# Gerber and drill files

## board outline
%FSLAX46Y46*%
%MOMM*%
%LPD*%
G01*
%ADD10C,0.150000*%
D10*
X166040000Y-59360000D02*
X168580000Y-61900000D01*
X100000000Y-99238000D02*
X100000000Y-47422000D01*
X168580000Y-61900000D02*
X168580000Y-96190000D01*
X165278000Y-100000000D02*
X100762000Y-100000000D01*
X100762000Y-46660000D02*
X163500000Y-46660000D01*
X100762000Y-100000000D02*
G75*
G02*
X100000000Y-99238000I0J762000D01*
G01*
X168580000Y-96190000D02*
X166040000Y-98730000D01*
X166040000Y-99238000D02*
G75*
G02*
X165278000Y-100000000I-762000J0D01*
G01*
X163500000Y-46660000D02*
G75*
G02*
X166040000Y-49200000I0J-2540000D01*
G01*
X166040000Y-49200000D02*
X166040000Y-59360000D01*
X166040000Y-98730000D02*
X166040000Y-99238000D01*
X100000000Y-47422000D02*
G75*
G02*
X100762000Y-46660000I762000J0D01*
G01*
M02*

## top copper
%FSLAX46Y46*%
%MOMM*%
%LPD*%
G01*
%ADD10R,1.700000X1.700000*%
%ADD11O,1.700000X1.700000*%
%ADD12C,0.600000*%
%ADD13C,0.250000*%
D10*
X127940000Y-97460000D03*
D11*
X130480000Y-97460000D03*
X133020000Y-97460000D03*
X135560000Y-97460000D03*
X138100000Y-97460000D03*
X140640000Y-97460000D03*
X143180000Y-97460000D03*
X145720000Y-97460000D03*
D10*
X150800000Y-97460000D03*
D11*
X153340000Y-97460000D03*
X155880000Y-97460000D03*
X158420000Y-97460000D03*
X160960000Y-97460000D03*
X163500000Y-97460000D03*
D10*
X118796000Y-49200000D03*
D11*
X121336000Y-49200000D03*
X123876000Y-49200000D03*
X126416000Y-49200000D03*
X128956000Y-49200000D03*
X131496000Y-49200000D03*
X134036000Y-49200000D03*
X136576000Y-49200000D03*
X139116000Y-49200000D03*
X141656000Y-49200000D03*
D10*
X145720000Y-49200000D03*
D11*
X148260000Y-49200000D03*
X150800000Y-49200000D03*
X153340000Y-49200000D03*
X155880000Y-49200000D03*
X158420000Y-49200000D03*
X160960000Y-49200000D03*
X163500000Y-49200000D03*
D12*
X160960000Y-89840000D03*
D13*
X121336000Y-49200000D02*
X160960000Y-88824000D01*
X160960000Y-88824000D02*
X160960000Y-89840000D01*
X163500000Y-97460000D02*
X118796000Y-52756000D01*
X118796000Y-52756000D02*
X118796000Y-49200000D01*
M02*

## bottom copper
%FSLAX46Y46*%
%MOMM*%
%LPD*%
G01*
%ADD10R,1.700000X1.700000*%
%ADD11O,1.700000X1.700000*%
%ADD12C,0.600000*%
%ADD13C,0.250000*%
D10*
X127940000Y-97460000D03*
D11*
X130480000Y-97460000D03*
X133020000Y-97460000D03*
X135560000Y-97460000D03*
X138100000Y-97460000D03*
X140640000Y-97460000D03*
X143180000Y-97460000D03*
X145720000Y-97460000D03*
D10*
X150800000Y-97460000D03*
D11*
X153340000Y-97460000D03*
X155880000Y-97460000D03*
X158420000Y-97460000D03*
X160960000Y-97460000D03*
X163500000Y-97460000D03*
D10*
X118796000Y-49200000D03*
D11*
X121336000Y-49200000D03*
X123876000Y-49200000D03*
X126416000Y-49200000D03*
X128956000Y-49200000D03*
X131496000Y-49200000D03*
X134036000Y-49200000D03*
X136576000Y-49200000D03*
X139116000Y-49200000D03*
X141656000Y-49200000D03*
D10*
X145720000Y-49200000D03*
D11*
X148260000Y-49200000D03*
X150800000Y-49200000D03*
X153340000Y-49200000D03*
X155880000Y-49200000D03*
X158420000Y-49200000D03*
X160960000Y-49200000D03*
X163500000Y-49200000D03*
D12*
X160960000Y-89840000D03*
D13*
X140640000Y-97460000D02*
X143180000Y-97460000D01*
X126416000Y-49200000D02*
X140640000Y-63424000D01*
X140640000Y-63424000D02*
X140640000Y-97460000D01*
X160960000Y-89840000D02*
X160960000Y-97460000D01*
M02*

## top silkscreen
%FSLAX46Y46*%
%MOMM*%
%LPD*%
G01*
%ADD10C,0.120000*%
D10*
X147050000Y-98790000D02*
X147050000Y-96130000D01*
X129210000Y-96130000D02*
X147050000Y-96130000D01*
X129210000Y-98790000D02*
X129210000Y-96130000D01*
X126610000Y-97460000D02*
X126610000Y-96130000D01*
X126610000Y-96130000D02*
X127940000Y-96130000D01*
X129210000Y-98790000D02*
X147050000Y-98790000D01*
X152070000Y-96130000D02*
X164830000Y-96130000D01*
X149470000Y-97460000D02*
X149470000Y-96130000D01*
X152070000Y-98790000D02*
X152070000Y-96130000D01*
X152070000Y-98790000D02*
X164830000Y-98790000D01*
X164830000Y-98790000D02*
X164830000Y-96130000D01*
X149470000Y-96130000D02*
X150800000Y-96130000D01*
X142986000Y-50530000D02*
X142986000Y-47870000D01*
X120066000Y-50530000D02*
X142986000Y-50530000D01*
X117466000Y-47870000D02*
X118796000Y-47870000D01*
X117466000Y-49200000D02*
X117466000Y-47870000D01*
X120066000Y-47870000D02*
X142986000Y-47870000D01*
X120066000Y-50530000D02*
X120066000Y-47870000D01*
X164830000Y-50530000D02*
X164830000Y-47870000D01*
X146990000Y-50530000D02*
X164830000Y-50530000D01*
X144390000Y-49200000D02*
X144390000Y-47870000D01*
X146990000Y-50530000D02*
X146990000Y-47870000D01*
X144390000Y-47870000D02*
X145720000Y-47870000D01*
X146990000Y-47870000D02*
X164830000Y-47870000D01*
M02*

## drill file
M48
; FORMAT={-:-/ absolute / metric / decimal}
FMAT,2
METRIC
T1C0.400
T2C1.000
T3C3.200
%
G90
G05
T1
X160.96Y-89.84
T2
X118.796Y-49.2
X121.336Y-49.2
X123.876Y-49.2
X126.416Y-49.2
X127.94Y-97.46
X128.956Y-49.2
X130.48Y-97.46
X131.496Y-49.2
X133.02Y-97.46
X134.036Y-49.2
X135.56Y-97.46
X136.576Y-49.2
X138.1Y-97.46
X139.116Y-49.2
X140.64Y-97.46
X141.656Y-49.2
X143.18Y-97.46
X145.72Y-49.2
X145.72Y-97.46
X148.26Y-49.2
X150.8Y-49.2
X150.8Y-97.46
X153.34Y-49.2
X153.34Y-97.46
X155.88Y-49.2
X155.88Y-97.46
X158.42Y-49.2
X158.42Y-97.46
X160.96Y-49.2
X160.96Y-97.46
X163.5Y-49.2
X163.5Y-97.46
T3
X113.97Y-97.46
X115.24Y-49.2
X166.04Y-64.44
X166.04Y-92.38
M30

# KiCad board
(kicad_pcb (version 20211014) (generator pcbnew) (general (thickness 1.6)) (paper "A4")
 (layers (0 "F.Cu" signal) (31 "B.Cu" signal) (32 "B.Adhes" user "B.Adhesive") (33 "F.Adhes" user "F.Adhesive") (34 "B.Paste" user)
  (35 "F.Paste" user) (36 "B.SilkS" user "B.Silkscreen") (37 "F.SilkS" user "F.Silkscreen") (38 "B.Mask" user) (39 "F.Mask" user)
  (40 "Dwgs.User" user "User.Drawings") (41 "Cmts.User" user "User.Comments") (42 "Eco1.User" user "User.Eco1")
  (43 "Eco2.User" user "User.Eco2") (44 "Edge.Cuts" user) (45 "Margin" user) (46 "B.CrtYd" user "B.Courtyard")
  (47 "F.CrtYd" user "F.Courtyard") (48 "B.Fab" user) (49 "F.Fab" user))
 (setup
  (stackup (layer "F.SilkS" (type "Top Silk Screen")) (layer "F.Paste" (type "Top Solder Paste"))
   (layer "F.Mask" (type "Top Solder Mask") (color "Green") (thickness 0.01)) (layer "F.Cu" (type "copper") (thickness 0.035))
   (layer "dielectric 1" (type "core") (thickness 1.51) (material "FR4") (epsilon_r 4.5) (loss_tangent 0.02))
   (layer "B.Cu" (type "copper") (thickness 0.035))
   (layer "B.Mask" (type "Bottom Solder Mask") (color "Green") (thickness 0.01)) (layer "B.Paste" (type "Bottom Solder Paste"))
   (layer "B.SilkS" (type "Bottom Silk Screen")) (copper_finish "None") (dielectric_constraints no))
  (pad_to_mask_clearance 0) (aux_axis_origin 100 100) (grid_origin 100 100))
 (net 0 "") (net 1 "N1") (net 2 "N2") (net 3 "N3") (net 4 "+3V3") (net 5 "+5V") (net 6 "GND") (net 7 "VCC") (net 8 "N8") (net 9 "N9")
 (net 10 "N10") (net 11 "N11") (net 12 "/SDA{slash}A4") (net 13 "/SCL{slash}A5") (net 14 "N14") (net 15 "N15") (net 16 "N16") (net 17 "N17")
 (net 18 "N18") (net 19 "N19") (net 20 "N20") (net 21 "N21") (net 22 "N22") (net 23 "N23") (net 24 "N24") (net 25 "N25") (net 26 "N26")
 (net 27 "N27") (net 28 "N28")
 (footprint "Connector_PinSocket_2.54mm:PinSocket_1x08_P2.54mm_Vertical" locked (layer "F.Cu") (at 127.94 97.46 90)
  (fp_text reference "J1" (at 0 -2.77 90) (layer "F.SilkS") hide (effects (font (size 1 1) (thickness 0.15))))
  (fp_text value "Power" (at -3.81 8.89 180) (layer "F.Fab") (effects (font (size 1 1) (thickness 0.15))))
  (fp_line (start -1.33 19.11) (end 1.33 19.11) (layer "F.SilkS") (width 0.12))
  (fp_line (start 1.33 1.27) (end 1.33 19.11) (layer "F.SilkS") (width 0.12))
  (fp_line (start -1.33 1.27) (end 1.33 1.27) (layer "F.SilkS") (width 0.12))
  (fp_line (start 0 -1.33) (end 1.33 -1.33) (layer "F.SilkS") (width 0.12))
  (fp_line (start 1.33 -1.33) (end 1.33 0) (layer "F.SilkS") (width 0.12))
  (fp_line (start -1.33 1.27) (end -1.33 19.11) (layer "F.SilkS") (width 0.12))
  (pad "1" thru_hole rect locked (at 0 0 90) (size 1.7 1.7) (drill 1) (layers *.Cu *.Mask) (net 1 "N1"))
  (pad "2" thru_hole oval locked (at 0 2.54 90) (size 1.7 1.7) (drill 1) (layers *.Cu *.Mask) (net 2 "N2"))
  (pad "3" thru_hole oval locked (at 0 5.08 90) (size 1.7 1.7) (drill 1) (layers *.Cu *.Mask) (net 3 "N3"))
  (pad "4" thru_hole oval locked (at 0 7.62 90) (size 1.7 1.7) (drill 1) (layers *.Cu *.Mask) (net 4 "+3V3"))
  (pad "5" thru_hole oval locked (at 0 10.16 90) (size 1.7 1.7) (drill 1) (layers *.Cu *.Mask) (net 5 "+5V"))
  (pad "6" thru_hole oval locked (at 0 12.7 90) (size 1.7 1.7) (drill 1) (layers *.Cu *.Mask) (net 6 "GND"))
  (pad "7" thru_hole oval locked (at 0 15.24 90) (size 1.7 1.7) (drill 1) (layers *.Cu *.Mask) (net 6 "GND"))
  (pad "8" thru_hole oval locked (at 0 17.78 90) (size 1.7 1.7) (drill 1) (layers *.Cu *.Mask) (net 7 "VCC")))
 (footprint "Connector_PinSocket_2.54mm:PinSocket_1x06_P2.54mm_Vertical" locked (layer "F.Cu") (at 150.8 97.46 90)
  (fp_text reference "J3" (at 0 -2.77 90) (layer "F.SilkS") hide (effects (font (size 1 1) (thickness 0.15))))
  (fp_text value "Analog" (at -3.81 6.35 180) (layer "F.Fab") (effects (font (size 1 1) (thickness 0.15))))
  (fp_line (start 1.33 1.27) (end 1.33 14.03) (layer "F.SilkS") (width 0.12))
  (fp_line (start 0 -1.33) (end 1.33 -1.33) (layer "F.SilkS") (width 0.12))
  (fp_line (start -1.33 1.27) (end 1.33 1.27) (layer "F.SilkS") (width 0.12))
  (fp_line (start -1.33 1.27) (end -1.33 14.03) (layer "F.SilkS") (width 0.12))
  (fp_line (start -1.33 14.03) (end 1.33 14.03) (layer "F.SilkS") (width 0.12))
  (fp_line (start 1.33 -1.33) (end 1.33 0) (layer "F.SilkS") (width 0.12))
  (pad "1" thru_hole rect locked (at 0 0 90) (size 1.7 1.7) (drill 1) (layers *.Cu *.Mask) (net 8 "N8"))
  (pad "2" thru_hole oval locked (at 0 2.54 90) (size 1.7 1.7) (drill 1) (layers *.Cu *.Mask) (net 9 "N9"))
  (pad "3" thru_hole oval locked (at 0 5.08 90) (size 1.7 1.7) (drill 1) (layers *.Cu *.Mask) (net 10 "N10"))
  (pad "4" thru_hole oval locked (at 0 7.62 90) (size 1.7 1.7) (drill 1) (layers *.Cu *.Mask) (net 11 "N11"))
  (pad "5" thru_hole oval locked (at 0 10.16 90) (size 1.7 1.7) (drill 1) (layers *.Cu *.Mask) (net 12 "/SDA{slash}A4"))
  (pad "6" thru_hole oval locked (at 0 12.7 90) (size 1.7 1.7) (drill 1) (layers *.Cu *.Mask) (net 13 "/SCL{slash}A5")))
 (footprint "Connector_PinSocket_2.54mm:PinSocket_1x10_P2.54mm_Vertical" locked (layer "F.Cu") (at 118.796 49.2 90)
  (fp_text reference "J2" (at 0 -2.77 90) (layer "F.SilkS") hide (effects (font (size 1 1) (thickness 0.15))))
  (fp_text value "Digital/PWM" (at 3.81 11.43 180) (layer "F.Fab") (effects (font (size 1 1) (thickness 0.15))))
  (fp_line (start -1.33 24.19) (end 1.33 24.19) (layer "F.SilkS") (width 0.12))
  (fp_line (start -1.33 1.27) (end -1.33 24.19) (layer "F.SilkS") (width 0.12))
  (fp_line (start 1.33 -1.33) (end 1.33 0) (layer "F.SilkS") (width 0.12))
  (fp_line (start 0 -1.33) (end 1.33 -1.33) (layer "F.SilkS") (width 0.12))
  (fp_line (start 1.33 1.27) (end 1.33 24.19) (layer "F.SilkS") (width 0.12))
  (fp_line (start -1.33 1.27) (end 1.33 1.27) (layer "F.SilkS") (width 0.12))
  (pad "1" thru_hole rect locked (at 0 0 90) (size 1.7 1.7) (drill 1) (layers *.Cu *.Mask) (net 13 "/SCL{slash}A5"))
  (pad "2" thru_hole oval locked (at 0 2.54 90) (size 1.7 1.7) (drill 1) (layers *.Cu *.Mask) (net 12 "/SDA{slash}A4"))
  (pad "3" thru_hole oval locked (at 0 5.08 90) (size 1.7 1.7) (drill 1) (layers *.Cu *.Mask) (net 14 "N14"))
  (pad "4" thru_hole oval locked (at 0 7.62 90) (size 1.7 1.7) (drill 1) (layers *.Cu *.Mask) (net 6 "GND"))
  (pad "5" thru_hole oval locked (at 0 10.16 90) (size 1.7 1.7) (drill 1) (layers *.Cu *.Mask) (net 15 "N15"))
  (pad "6" thru_hole oval locked (at 0 12.7 90) (size 1.7 1.7) (drill 1) (layers *.Cu *.Mask) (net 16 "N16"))
  (pad "7" thru_hole oval locked (at 0 15.24 90) (size 1.7 1.7) (drill 1) (layers *.Cu *.Mask) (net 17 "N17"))
  (pad "8" thru_hole oval locked (at 0 17.78 90) (size 1.7 1.7) (drill 1) (layers *.Cu *.Mask) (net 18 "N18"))
  (pad "9" thru_hole oval locked (at 0 20.32 90) (size 1.7 1.7) (drill 1) (layers *.Cu *.Mask) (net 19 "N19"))
  (pad "10" thru_hole oval locked (at 0 22.86 90) (size 1.7 1.7) (drill 1) (layers *.Cu *.Mask) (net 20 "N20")))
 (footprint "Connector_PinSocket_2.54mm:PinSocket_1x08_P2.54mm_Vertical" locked (layer "F.Cu") (at 145.72 49.2 90)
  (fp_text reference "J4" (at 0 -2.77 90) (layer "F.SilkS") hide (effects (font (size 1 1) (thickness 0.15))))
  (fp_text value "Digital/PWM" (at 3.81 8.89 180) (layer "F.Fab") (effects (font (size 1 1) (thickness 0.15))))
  (fp_line (start -1.33 19.11) (end 1.33 19.11) (layer "F.SilkS") (width 0.12))
  (fp_line (start -1.33 1.27) (end -1.33 19.11) (layer "F.SilkS") (width 0.12))
  (fp_line (start 0 -1.33) (end 1.33 -1.33) (layer "F.SilkS") (width 0.12))
  (fp_line (start -1.33 1.27) (end 1.33 1.27) (layer "F.SilkS") (width 0.12))
  (fp_line (start 1.33 -1.33) (end 1.33 0) (layer "F.SilkS") (width 0.12))
  (fp_line (start 1.33 1.27) (end 1.33 19.11) (layer "F.SilkS") (width 0.12))
  (pad "1" thru_hole rect locked (at 0 0 90) (size 1.7 1.7) (drill 1) (layers *.Cu *.Mask) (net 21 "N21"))
  (pad "2" thru_hole oval locked (at 0 2.54 90) (size 1.7 1.7) (drill 1) (layers *.Cu *.Mask) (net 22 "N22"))
  (pad "3" thru_hole oval locked (at 0 5.08 90) (size 1.7 1.7) (drill 1) (layers *.Cu *.Mask) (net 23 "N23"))
  (pad "4" thru_hole oval locked (at 0 7.62 90) (size 1.7 1.7) (drill 1) (layers *.Cu *.Mask) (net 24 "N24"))
  (pad "5" thru_hole oval locked (at 0 10.16 90) (size 1.7 1.7) (drill 1) (layers *.Cu *.Mask) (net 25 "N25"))
  (pad "6" thru_hole oval locked (at 0 12.7 90) (size 1.7 1.7) (drill 1) (layers *.Cu *.Mask) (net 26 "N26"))
  (pad "7" thru_hole oval locked (at 0 15.24 90) (size 1.7 1.7) (drill 1) (layers *.Cu *.Mask) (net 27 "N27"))
  (pad "8" thru_hole oval locked (at 0 17.78 90) (size 1.7 1.7) (drill 1) (layers *.Cu *.Mask) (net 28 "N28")))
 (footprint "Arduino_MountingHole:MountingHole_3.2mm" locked (layer "F.Cu") (at 115.24 49.2)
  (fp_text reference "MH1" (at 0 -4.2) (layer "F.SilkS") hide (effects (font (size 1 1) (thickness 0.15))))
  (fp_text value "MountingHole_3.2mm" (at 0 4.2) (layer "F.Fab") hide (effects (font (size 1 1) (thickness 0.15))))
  (pad "" np_thru_hole circle locked (at 0 0) (size 3.2 3.2) (drill 3.2) (layers *.Cu *.Mask)))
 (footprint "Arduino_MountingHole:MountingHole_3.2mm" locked (layer "F.Cu") (at 113.97 97.46)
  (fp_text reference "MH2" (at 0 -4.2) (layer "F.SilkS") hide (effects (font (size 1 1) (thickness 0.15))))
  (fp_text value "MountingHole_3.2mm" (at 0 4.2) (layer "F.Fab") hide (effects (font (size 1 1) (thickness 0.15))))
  (pad "" np_thru_hole circle locked (at 0 0) (size 3.2 3.2) (drill 3.2) (layers *.Cu *.Mask)))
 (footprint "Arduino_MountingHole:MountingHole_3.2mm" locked (layer "F.Cu") (at 166.04 64.44)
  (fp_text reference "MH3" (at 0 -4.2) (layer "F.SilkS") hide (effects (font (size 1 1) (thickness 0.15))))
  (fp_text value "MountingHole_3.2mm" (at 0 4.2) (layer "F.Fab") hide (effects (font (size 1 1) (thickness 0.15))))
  (pad "" np_thru_hole circle locked (at 0 0) (size 3.2 3.2) (drill 3.2) (layers *.Cu *.Mask)))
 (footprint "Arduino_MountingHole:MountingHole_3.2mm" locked (layer "F.Cu") (at 166.04 92.38)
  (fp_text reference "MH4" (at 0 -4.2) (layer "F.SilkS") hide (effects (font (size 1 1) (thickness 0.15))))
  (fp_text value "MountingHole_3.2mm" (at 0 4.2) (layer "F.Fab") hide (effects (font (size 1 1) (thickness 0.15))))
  (pad "" np_thru_hole circle locked (at 0 0) (size 3.2 3.2) (drill 3.2) (layers *.Cu *.Mask)))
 (gr_line (start 166.04 59.36) (end 168.58 61.9) (layer "Edge.Cuts") (width 0.15))
 (gr_line (start 100 99.238) (end 100 47.422) (layer "Edge.Cuts") (width 0.15))
 (gr_line (start 168.58 61.9) (end 168.58 96.19) (layer "Edge.Cuts") (width 0.15))
 (gr_line (start 165.278 100) (end 100.762 100) (layer "Edge.Cuts") (width 0.15))
 (gr_line (start 100.762 46.66) (end 163.5 46.66) (layer "Edge.Cuts") (width 0.15))
 (gr_arc (start 100.762 100) (mid 100.223185 99.776815) (end 100 99.238) (layer "Edge.Cuts") (width 0.15))
 (gr_line (start 168.58 96.19) (end 166.04 98.73) (layer "Edge.Cuts") (width 0.15))
 (gr_arc (start 166.04 99.238) (mid 165.816815 99.776815) (end 165.278 100) (layer "Edge.Cuts") (width 0.15))
 (gr_arc (start 163.5 46.66) (mid 165.296051 47.403949) (end 166.04 49.2) (layer "Edge.Cuts") (width 0.15))
 (gr_line (start 166.04 49.2) (end 166.04 59.36) (layer "Edge.Cuts") (width 0.15))
 (gr_line (start 166.04 98.73) (end 166.04 99.238) (layer "Edge.Cuts") (width 0.15))
 (gr_arc (start 100 47.422) (mid 100.223185 46.883185) (end 100.762 46.66) (layer "Edge.Cuts") (width 0.15))
 (segment (start 140.64 97.46) (end 143.18 97.46) (width 0.25) (layer "B.Cu") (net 6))
 (segment (start 126.416 49.2) (end 140.64 63.424) (width 0.25) (layer "B.Cu") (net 6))
 (segment (start 140.64 63.424) (end 140.64 97.46) (width 0.25) (layer "B.Cu") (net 6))
 (segment (start 121.336 49.2) (end 160.96 88.824) (width 0.25) (layer "F.Cu") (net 12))
 (segment (start 160.96 88.824) (end 160.96 89.84) (width 0.25) (layer "F.Cu") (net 12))
 (via (at 160.96 89.84) (size 0.6) (drill 0.4) (layers "F.Cu" "B.Cu") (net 12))
 (segment (start 160.96 89.84) (end 160.96 97.46) (width 0.25) (layer "B.Cu") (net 12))
 (segment (start 163.5 97.46) (end 118.796 52.756) (width 0.25) (layer "F.Cu") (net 13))
 (segment (start 118.796 52.756) (end 118.796 49.2) (width 0.25) (layer "F.Cu") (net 13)))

